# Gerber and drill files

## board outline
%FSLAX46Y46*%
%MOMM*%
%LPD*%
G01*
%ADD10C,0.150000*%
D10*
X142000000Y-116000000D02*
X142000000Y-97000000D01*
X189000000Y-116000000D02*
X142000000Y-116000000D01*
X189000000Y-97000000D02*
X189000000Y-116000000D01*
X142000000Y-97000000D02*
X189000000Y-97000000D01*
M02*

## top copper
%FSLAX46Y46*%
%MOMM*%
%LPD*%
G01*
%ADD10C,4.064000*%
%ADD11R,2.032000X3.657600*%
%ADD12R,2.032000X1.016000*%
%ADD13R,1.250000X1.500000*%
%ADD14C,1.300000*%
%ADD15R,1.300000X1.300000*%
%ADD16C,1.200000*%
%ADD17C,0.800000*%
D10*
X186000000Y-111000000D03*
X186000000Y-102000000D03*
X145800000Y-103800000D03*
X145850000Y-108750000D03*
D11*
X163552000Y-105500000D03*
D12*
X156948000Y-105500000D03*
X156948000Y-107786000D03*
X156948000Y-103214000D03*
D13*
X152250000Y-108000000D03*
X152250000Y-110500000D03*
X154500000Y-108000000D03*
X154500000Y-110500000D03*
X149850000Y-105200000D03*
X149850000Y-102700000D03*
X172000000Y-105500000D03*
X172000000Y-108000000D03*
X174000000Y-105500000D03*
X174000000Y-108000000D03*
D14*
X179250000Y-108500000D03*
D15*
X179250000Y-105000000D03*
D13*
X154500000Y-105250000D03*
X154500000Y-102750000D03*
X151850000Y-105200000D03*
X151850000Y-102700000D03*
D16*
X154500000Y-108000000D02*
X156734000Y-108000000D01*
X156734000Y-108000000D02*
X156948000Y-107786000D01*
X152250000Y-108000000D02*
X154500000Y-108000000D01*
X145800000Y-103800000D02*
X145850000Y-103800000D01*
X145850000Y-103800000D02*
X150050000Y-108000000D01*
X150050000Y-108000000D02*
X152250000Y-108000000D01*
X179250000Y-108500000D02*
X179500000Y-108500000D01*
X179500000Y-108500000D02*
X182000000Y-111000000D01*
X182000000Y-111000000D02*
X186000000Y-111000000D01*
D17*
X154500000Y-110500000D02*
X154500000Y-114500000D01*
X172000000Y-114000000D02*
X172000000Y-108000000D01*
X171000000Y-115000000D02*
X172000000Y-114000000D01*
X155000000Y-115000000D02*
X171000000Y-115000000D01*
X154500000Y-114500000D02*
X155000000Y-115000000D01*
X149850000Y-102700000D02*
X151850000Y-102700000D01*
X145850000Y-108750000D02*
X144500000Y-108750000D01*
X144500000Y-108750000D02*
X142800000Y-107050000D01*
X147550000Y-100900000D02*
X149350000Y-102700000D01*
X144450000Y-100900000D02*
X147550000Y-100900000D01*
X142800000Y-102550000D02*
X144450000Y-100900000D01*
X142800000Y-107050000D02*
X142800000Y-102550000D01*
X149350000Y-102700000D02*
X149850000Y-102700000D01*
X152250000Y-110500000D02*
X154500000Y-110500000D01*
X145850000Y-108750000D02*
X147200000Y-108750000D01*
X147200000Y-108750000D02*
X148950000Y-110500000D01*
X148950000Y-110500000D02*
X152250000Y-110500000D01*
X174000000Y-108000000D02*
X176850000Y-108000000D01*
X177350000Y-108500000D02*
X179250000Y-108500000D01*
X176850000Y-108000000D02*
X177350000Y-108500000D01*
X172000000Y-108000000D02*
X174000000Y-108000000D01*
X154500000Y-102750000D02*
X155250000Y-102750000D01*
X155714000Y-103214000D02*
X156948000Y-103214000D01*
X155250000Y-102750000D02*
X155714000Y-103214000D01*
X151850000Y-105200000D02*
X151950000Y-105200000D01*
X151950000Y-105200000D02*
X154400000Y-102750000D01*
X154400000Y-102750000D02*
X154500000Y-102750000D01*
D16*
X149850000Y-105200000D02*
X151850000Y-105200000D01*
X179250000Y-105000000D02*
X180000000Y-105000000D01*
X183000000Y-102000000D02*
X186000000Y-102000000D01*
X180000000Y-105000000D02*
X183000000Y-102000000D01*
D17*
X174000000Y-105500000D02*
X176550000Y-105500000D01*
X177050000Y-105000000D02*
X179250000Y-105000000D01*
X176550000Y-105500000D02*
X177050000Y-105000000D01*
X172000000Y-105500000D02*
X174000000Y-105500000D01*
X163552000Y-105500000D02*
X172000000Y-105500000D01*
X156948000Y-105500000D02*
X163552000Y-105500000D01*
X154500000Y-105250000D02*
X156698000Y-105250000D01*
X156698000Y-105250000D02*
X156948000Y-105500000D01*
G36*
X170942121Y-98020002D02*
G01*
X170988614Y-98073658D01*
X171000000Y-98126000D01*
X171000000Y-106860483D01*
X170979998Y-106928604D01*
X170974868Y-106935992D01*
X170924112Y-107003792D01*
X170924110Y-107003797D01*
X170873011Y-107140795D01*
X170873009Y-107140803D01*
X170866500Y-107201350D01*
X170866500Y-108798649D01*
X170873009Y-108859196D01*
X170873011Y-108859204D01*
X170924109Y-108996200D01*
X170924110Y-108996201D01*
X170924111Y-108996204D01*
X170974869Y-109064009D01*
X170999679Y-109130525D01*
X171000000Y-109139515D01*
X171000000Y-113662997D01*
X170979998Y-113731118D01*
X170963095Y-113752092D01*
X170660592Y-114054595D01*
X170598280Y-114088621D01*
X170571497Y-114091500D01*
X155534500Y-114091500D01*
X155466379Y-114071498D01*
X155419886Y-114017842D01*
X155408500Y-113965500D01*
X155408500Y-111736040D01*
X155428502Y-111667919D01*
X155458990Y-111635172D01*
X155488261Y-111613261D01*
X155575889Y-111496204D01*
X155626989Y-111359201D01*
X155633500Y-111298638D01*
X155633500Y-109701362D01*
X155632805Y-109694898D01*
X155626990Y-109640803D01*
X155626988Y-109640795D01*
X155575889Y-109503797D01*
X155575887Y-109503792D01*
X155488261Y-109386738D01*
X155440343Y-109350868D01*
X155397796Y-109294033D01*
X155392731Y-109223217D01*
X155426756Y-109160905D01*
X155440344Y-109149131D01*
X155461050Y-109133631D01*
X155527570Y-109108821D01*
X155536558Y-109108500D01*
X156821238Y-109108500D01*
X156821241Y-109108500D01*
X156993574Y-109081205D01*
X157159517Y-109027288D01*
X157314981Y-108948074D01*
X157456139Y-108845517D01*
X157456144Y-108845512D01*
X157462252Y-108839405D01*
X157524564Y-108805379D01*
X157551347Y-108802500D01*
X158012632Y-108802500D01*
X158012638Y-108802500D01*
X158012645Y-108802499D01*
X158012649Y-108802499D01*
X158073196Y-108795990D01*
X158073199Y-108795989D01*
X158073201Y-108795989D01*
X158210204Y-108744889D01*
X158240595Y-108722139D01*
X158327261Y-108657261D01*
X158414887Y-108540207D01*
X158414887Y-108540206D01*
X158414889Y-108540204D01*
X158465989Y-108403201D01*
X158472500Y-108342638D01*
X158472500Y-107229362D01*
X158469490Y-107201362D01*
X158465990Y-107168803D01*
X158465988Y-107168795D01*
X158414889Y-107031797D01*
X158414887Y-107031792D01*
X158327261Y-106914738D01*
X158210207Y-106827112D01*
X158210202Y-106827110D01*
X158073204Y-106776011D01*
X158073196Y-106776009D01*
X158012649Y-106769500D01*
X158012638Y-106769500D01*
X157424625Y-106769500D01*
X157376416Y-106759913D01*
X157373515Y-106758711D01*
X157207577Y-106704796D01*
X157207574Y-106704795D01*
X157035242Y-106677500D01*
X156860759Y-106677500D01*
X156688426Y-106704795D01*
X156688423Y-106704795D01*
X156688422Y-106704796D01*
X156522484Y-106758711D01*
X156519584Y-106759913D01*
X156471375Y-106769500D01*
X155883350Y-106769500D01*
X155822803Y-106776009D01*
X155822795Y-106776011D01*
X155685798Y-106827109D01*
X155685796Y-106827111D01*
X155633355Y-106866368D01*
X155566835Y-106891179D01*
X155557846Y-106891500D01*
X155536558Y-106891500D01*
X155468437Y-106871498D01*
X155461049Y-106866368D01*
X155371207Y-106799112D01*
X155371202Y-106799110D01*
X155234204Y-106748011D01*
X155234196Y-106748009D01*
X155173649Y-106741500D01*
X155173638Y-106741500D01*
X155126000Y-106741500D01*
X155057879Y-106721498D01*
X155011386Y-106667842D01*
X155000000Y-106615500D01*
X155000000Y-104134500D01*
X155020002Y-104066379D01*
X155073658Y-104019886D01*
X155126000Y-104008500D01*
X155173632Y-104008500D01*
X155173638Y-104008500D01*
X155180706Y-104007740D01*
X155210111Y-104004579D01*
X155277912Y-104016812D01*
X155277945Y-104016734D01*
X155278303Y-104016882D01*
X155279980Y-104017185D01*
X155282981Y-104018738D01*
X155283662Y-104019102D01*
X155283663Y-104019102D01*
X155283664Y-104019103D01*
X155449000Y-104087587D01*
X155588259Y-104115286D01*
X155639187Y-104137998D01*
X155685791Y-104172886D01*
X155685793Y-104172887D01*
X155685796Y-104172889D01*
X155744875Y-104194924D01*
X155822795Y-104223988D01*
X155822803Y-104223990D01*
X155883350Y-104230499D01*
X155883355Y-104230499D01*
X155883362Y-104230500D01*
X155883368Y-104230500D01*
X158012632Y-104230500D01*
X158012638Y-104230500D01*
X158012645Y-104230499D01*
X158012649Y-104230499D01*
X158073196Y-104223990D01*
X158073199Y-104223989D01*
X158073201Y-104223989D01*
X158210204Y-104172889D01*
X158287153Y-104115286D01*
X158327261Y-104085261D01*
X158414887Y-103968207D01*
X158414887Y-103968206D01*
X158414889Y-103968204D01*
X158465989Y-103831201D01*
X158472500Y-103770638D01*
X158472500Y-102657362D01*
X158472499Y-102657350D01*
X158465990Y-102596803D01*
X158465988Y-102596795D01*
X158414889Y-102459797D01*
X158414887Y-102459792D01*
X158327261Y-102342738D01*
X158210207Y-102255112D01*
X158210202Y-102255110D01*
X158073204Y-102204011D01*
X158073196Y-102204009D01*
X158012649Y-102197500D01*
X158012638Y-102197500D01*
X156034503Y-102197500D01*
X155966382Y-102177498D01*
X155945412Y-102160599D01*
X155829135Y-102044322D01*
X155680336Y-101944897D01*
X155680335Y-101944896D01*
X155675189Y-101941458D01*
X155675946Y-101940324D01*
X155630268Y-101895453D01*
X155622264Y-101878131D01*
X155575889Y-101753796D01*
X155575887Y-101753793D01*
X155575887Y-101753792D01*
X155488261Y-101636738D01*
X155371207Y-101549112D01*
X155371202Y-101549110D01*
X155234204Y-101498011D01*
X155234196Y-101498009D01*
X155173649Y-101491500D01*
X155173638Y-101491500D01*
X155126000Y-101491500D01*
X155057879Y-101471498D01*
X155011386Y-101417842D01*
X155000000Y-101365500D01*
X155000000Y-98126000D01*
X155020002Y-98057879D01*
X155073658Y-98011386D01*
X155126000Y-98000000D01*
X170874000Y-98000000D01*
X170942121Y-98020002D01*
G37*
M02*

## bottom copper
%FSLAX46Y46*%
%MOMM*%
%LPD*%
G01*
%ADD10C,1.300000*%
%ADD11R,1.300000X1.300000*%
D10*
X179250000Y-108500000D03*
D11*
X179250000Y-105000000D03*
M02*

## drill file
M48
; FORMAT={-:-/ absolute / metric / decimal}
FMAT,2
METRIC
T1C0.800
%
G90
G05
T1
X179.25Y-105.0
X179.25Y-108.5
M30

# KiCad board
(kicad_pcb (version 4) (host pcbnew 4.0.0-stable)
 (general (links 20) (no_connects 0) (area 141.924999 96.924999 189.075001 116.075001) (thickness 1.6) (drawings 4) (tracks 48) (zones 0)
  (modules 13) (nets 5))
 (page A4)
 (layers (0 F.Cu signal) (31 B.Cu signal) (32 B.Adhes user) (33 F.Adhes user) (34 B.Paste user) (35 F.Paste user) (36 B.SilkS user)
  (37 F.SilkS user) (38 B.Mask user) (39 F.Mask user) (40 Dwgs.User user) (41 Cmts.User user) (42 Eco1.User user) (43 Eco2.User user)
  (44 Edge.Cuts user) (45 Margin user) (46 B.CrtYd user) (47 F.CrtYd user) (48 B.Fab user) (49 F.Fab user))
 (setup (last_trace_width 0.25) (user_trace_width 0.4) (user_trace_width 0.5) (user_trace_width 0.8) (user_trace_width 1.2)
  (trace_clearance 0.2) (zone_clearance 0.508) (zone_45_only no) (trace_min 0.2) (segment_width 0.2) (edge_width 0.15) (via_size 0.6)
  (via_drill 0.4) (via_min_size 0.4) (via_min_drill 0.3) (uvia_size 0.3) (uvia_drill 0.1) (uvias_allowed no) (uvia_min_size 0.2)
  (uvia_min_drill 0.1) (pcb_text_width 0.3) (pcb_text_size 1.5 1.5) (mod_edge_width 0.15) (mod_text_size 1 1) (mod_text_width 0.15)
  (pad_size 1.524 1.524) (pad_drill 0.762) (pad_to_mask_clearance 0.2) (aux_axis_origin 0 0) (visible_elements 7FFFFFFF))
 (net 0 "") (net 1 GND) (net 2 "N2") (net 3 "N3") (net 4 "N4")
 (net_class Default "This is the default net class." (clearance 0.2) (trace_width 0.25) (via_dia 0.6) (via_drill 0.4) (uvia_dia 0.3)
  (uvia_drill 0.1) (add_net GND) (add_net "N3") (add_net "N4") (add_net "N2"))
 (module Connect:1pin (layer F.Cu) (at 186 111)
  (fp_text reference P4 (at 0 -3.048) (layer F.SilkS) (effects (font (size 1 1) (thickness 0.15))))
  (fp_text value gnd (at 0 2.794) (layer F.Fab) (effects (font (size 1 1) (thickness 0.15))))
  (pad 1 smd circle (at 0 0) (size 4.064 4.064) (layers F.Cu F.Paste F.Mask) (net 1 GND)))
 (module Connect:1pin (layer F.Cu) (at 186 102)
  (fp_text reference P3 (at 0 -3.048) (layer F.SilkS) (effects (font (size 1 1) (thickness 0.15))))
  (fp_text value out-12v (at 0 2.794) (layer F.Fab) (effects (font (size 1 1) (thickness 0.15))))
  (pad 1 smd circle (at 0 0) (size 4.064 4.064) (layers F.Cu F.Paste F.Mask) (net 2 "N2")))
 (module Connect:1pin (layer F.Cu) (at 145.8 103.8)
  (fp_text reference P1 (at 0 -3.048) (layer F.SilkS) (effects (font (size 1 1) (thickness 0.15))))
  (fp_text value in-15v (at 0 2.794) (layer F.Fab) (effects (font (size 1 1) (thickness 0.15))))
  (pad 1 smd circle (at 0 0) (size 4.064 4.064) (layers F.Cu F.Paste F.Mask) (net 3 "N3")))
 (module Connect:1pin (layer F.Cu) (at 145.85 108.75)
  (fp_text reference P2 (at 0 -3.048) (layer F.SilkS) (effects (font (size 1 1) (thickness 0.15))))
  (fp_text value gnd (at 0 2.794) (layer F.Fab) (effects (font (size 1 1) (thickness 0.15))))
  (pad 1 smd circle (at 0 0) (size 4.064 4.064) (layers F.Cu F.Paste F.Mask) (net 1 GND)))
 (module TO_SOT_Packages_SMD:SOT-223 (layer F.Cu) (at 160.25 105.5 270)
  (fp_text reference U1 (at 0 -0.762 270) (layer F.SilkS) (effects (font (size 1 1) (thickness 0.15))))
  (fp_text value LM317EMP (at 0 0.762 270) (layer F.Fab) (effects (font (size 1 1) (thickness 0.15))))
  (pad 2 smd rect (at 0 -3.302 270) (size 3.6576 2.032) (layers F.Cu F.Paste F.Mask) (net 2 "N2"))
  (pad 2 smd rect (at 0 3.302 270) (size 1.016 2.032) (layers F.Cu F.Paste F.Mask) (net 2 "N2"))
  (pad 3 smd rect (at 2.286 3.302 270) (size 1.016 2.032) (layers F.Cu F.Paste F.Mask) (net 3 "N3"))
  (pad 1 smd rect (at -2.286 3.302 270) (size 1.016 2.032) (layers F.Cu F.Paste F.Mask) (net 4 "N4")))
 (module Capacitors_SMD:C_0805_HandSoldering (layer F.Cu) (at 152.25 109.25 270)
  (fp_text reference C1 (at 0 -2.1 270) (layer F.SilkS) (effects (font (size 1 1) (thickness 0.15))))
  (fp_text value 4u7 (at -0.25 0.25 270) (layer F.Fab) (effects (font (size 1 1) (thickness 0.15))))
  (pad 1 smd rect (at -1.25 0 270) (size 1.5 1.25) (layers F.Cu F.Paste F.Mask) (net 3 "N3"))
  (pad 2 smd rect (at 1.25 0 270) (size 1.5 1.25) (layers F.Cu F.Paste F.Mask) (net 1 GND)))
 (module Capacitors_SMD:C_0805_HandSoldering (layer F.Cu) (at 154.5 109.25 270)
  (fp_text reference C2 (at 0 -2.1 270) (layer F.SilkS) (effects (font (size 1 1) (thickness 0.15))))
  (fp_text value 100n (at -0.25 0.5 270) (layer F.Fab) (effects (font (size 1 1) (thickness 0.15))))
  (pad 1 smd rect (at -1.25 0 270) (size 1.5 1.25) (layers F.Cu F.Paste F.Mask) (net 3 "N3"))
  (pad 2 smd rect (at 1.25 0 270) (size 1.5 1.25) (layers F.Cu F.Paste F.Mask) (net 1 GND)))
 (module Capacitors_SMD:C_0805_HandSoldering (layer F.Cu) (at 149.85 103.95 90)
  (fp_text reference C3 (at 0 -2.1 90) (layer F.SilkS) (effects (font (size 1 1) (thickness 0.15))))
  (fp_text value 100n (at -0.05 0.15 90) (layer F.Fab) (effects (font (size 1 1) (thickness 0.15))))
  (pad 1 smd rect (at -1.25 0 90) (size 1.5 1.25) (layers F.Cu F.Paste F.Mask) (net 4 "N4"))
  (pad 2 smd rect (at 1.25 0 90) (size 1.5 1.25) (layers F.Cu F.Paste F.Mask) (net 1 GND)))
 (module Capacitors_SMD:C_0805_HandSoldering (layer F.Cu) (at 172 106.75 270)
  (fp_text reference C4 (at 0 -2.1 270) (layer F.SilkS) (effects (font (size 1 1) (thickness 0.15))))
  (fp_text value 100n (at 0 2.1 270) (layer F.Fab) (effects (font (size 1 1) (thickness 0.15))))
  (pad 1 smd rect (at -1.25 0 270) (size 1.5 1.25) (layers F.Cu F.Paste F.Mask) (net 2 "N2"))
  (pad 2 smd rect (at 1.25 0 270) (size 1.5 1.25) (layers F.Cu F.Paste F.Mask) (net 1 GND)))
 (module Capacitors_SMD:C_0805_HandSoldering (layer F.Cu) (at 174 106.75 270)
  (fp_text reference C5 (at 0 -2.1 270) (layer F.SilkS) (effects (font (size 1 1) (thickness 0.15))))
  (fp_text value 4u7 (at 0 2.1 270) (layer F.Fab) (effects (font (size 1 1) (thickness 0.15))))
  (pad 1 smd rect (at -1.25 0 270) (size 1.5 1.25) (layers F.Cu F.Paste F.Mask) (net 2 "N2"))
  (pad 2 smd rect (at 1.25 0 270) (size 1.5 1.25) (layers F.Cu F.Paste F.Mask) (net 1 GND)))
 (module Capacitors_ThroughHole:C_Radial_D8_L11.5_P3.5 (layer F.Cu) (at 179.25 105 270)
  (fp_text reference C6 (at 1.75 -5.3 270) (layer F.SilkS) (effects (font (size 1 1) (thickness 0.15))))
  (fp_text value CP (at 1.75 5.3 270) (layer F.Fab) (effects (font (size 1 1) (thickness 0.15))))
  (pad 2 thru_hole circle (at 3.5 0 270) (size 1.3 1.3) (drill 0.8) (layers *.Cu *.Mask F.SilkS) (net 1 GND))
  (pad 1 thru_hole rect (at 0 0 270) (size 1.3 1.3) (drill 0.8) (layers *.Cu *.Mask F.SilkS) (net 2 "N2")))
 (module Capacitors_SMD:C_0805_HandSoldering (layer F.Cu) (at 154.5 104 90)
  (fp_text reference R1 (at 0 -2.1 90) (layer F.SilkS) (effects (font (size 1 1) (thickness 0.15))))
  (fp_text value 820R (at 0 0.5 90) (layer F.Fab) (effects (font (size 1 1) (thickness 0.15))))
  (pad 1 smd rect (at -1.25 0 90) (size 1.5 1.25) (layers F.Cu F.Paste F.Mask) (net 2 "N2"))
  (pad 2 smd rect (at 1.25 0 90) (size 1.5 1.25) (layers F.Cu F.Paste F.Mask) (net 4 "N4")))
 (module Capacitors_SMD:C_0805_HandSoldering (layer F.Cu) (at 151.85 103.95 90)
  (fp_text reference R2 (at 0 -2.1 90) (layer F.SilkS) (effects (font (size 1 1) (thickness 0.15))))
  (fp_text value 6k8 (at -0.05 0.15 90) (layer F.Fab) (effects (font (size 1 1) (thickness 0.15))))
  (pad 1 smd rect (at -1.25 0 90) (size 1.5 1.25) (layers F.Cu F.Paste F.Mask) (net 4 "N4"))
  (pad 2 smd rect (at 1.25 0 90) (size 1.5 1.25) (layers F.Cu F.Paste F.Mask) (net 1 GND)))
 (gr_line (start 142 116) (end 142 97) (angle 90) (layer Edge.Cuts) (width 0.15))
 (gr_line (start 189 116) (end 142 116) (angle 90) (layer Edge.Cuts) (width 0.15))
 (gr_line (start 189 97) (end 189 116) (angle 90) (layer Edge.Cuts) (width 0.15))
 (gr_line (start 142 97) (end 189 97) (angle 90) (layer Edge.Cuts) (width 0.15))
 (segment (start 154.5 108) (end 156.734 108) (width 1.2) (layer F.Cu) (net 3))
 (segment (start 156.734 108) (end 156.948 107.786) (width 1.2) (layer F.Cu) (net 3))
 (segment (start 152.25 108) (end 154.5 108) (width 1.2) (layer F.Cu) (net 3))
 (segment (start 145.8 103.8) (end 145.85 103.8) (width 1.2) (layer F.Cu) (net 3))
 (segment (start 145.85 103.8) (end 150.05 108) (width 1.2) (layer F.Cu) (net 3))
 (segment (start 150.05 108) (end 152.25 108) (width 1.2) (layer F.Cu) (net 3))
 (segment (start 179.25 108.5) (end 179.5 108.5) (width 1.2) (layer F.Cu) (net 1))
 (segment (start 179.5 108.5) (end 182 111) (width 1.2) (layer F.Cu) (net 1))
 (segment (start 182 111) (end 186 111) (width 1.2) (layer F.Cu) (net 1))
 (segment (start 154.5 110.5) (end 154.5 114.5) (width 0.8) (layer F.Cu) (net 1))
 (segment (start 172 114) (end 172 108) (width 0.8) (layer F.Cu) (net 1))
 (segment (start 171 115) (end 172 114) (width 0.8) (layer F.Cu) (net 1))
 (segment (start 155 115) (end 171 115) (width 0.8) (layer F.Cu) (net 1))
 (segment (start 154.5 114.5) (end 155 115) (width 0.8) (layer F.Cu) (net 1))
 (segment (start 149.85 102.7) (end 151.85 102.7) (width 0.8) (layer F.Cu) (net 1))
 (segment (start 145.85 108.75) (end 144.5 108.75) (width 0.8) (layer F.Cu) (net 1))
 (segment (start 144.5 108.75) (end 142.8 107.05) (width 0.8) (layer F.Cu) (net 1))
 (segment (start 147.55 100.9) (end 149.35 102.7) (width 0.8) (layer F.Cu) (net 1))
 (segment (start 144.45 100.9) (end 147.55 100.9) (width 0.8) (layer F.Cu) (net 1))
 (segment (start 142.8 102.55) (end 144.45 100.9) (width 0.8) (layer F.Cu) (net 1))
 (segment (start 142.8 107.05) (end 142.8 102.55) (width 0.8) (layer F.Cu) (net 1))
 (segment (start 149.35 102.7) (end 149.85 102.7) (width 0.8) (layer F.Cu) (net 1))
 (segment (start 152.25 110.5) (end 154.5 110.5) (width 0.8) (layer F.Cu) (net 1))
 (segment (start 145.85 108.75) (end 147.2 108.75) (width 0.8) (layer F.Cu) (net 1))
 (segment (start 147.2 108.75) (end 148.95 110.5) (width 0.8) (layer F.Cu) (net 1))
 (segment (start 148.95 110.5) (end 152.25 110.5) (width 0.8) (layer F.Cu) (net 1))
 (segment (start 174 108) (end 176.85 108) (width 0.8) (layer F.Cu) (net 1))
 (segment (start 177.35 108.5) (end 179.25 108.5) (width 0.8) (layer F.Cu) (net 1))
 (segment (start 176.85 108) (end 177.35 108.5) (width 0.8) (layer F.Cu) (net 1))
 (segment (start 172 108) (end 174 108) (width 0.8) (layer F.Cu) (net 1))
 (segment (start 154.5 102.75) (end 155.25 102.75) (width 0.8) (layer F.Cu) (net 4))
 (segment (start 155.714 103.214) (end 156.948 103.214) (width 0.8) (layer F.Cu) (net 4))
 (segment (start 155.25 102.75) (end 155.714 103.214) (width 0.8) (layer F.Cu) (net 4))
 (segment (start 151.85 105.2) (end 151.95 105.2) (width 0.8) (layer F.Cu) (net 4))
 (segment (start 151.95 105.2) (end 154.4 102.75) (width 0.8) (layer F.Cu) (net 4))
 (segment (start 154.4 102.75) (end 154.5 102.75) (width 0.8) (layer F.Cu) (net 4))
 (segment (start 149.85 105.2) (end 151.85 105.2) (width 1.2) (layer F.Cu) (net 4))
 (segment (start 179.25 105) (end 180 105) (width 1.2) (layer F.Cu) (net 2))
 (segment (start 183 102) (end 186 102) (width 1.2) (layer F.Cu) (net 2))
 (segment (start 180 105) (end 183 102) (width 1.2) (layer F.Cu) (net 2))
 (segment (start 174 105.5) (end 176.55 105.5) (width 0.8) (layer F.Cu) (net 2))
 (segment (start 177.05 105) (end 179.25 105) (width 0.8) (layer F.Cu) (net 2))
 (segment (start 176.55 105.5) (end 177.05 105) (width 0.8) (layer F.Cu) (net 2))
 (segment (start 172 105.5) (end 174 105.5) (width 0.8) (layer F.Cu) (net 2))
 (segment (start 163.552 105.5) (end 172 105.5) (width 0.8) (layer F.Cu) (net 2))
 (segment (start 156.948 105.5) (end 163.552 105.5) (width 0.8) (layer F.Cu) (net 2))
 (segment (start 154.5 105.25) (end 156.698 105.25) (width 0.8) (layer F.Cu) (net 2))
 (segment (start 156.698 105.25) (end 156.948 105.5) (width 0.8) (layer F.Cu) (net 2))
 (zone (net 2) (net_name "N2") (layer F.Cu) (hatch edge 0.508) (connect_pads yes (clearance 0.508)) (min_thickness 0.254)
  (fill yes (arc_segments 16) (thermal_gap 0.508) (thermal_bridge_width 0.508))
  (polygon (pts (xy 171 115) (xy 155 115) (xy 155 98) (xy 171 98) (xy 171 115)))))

